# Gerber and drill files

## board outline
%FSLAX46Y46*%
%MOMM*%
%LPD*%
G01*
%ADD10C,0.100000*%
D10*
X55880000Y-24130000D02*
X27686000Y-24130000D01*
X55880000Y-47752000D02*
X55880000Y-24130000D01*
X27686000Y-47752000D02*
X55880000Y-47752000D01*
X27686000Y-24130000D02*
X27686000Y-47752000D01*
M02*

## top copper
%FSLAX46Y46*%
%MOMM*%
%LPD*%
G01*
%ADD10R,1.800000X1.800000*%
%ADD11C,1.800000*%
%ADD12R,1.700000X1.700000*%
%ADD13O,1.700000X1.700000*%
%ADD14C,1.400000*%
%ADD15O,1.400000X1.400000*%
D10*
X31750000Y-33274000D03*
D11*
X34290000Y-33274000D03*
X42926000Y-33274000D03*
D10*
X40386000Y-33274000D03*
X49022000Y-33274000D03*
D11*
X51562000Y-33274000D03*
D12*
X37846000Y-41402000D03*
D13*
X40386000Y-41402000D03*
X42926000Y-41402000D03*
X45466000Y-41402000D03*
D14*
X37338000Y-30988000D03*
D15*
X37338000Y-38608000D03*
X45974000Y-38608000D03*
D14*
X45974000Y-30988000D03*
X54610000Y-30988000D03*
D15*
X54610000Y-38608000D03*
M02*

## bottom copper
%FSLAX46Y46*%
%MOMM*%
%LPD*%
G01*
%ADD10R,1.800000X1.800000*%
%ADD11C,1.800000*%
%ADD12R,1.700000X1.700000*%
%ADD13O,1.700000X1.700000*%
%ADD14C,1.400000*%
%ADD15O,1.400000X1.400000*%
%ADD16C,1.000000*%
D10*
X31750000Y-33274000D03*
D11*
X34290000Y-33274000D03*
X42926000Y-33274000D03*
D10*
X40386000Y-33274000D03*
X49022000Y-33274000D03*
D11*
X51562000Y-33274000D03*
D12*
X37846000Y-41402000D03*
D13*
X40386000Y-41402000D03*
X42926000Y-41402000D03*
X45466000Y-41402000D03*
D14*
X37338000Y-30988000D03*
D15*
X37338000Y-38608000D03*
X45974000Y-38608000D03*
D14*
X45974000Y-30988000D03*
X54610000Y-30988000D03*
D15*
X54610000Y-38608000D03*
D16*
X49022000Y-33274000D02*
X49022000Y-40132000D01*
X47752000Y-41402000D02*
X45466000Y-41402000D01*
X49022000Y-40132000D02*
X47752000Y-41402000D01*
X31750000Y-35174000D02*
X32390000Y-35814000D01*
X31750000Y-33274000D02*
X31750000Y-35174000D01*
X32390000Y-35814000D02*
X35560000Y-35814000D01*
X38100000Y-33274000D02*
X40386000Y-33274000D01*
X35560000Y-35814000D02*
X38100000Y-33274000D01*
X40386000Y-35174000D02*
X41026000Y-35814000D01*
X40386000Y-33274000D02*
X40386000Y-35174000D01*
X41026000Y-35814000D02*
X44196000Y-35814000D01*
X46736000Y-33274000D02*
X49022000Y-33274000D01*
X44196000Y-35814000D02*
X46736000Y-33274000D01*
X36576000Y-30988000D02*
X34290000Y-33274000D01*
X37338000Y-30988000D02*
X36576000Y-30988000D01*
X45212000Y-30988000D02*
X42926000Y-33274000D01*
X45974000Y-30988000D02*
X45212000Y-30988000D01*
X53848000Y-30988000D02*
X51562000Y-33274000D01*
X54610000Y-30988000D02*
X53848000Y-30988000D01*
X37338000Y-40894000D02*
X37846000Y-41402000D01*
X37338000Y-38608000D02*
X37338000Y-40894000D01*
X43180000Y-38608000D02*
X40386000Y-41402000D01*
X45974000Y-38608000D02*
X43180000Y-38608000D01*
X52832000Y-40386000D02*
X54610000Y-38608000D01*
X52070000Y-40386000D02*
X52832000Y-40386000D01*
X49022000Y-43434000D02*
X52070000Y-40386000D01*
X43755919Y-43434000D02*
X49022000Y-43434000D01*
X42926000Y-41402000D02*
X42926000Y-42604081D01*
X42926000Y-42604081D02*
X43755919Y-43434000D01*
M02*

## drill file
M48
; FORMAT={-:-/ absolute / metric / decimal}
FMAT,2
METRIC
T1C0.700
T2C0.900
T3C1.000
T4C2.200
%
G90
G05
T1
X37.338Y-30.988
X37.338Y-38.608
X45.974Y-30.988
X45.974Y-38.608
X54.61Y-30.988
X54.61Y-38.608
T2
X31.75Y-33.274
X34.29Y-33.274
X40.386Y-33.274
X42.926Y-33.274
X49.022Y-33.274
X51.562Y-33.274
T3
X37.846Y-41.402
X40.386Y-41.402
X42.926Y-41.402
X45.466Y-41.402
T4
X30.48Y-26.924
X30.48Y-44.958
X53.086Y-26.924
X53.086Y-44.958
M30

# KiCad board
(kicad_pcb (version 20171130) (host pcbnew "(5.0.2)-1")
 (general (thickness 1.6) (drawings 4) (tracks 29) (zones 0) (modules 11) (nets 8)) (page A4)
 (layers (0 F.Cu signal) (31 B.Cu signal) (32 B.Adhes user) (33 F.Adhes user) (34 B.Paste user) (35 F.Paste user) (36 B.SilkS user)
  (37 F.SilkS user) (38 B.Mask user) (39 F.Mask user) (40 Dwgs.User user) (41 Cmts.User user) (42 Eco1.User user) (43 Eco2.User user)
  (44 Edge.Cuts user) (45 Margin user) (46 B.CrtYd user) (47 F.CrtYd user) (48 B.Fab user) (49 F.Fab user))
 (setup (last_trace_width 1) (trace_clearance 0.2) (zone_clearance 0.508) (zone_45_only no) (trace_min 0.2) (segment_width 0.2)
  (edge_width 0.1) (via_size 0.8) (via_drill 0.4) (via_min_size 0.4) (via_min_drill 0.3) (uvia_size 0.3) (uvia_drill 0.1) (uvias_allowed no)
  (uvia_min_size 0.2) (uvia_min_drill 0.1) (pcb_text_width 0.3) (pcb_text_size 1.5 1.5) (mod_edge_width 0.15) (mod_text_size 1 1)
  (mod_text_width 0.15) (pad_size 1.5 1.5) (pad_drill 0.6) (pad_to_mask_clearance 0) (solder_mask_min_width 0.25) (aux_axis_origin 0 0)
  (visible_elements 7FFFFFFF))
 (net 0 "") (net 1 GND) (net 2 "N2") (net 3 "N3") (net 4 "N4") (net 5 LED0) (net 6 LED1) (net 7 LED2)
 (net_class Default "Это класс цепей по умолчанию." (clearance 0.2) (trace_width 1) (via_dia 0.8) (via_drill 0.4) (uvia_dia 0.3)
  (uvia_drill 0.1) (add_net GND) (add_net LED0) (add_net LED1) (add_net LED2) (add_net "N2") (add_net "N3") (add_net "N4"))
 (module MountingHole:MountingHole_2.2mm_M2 (layer F.Cu) (at 53.086 26.924)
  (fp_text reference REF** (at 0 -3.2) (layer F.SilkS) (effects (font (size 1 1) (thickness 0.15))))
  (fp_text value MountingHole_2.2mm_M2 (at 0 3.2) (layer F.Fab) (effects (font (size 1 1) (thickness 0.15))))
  (pad 1 np_thru_hole circle (at 0 0) (size 2.2 2.2) (drill 2.2) (layers *.Cu *.Mask)))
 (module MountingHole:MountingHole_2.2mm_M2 (layer F.Cu) (at 30.48 26.924)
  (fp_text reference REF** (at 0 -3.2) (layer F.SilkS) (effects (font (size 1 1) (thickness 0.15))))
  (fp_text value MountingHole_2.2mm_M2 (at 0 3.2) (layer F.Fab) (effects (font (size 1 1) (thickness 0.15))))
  (pad 1 np_thru_hole circle (at 0 0) (size 2.2 2.2) (drill 2.2) (layers *.Cu *.Mask)))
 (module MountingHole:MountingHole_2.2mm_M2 (layer F.Cu) (at 53.086 44.958)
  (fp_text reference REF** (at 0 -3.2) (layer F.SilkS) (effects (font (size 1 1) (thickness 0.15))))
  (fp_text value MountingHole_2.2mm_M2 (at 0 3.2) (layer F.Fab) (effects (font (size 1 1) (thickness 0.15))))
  (pad 1 np_thru_hole circle (at 0 0) (size 2.2 2.2) (drill 2.2) (layers *.Cu *.Mask)))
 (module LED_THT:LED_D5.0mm (layer F.Cu) (at 31.75 33.274)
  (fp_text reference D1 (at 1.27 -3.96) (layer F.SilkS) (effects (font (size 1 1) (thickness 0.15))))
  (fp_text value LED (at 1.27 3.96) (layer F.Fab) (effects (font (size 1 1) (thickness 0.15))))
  (pad 1 thru_hole rect (at 0 0) (size 1.8 1.8) (drill 0.9) (layers *.Cu *.Mask) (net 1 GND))
  (pad 2 thru_hole circle (at 2.54 0) (size 1.8 1.8) (drill 0.9) (layers *.Cu *.Mask) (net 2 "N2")))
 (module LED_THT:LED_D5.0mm (layer F.Cu) (at 40.386 33.274)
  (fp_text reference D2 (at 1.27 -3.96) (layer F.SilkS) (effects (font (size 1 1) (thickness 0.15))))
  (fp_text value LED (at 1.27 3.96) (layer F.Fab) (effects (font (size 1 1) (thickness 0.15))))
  (pad 2 thru_hole circle (at 2.54 0) (size 1.8 1.8) (drill 0.9) (layers *.Cu *.Mask) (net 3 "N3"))
  (pad 1 thru_hole rect (at 0 0) (size 1.8 1.8) (drill 0.9) (layers *.Cu *.Mask) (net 1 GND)))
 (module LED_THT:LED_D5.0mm (layer F.Cu) (at 49.022 33.274)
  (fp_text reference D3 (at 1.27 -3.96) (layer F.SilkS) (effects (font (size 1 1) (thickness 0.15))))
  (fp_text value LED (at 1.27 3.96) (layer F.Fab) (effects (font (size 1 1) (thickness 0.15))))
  (pad 1 thru_hole rect (at 0 0) (size 1.8 1.8) (drill 0.9) (layers *.Cu *.Mask) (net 1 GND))
  (pad 2 thru_hole circle (at 2.54 0) (size 1.8 1.8) (drill 0.9) (layers *.Cu *.Mask) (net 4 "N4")))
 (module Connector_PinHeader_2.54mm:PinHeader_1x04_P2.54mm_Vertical (layer F.Cu) (at 37.846 41.402 90)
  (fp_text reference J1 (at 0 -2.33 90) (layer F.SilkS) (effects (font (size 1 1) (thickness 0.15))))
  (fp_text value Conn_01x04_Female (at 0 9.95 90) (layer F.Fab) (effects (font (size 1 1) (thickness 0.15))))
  (pad 1 thru_hole rect (at 0 0 90) (size 1.7 1.7) (drill 1) (layers *.Cu *.Mask) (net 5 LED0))
  (pad 2 thru_hole oval (at 0 2.54 90) (size 1.7 1.7) (drill 1) (layers *.Cu *.Mask) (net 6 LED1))
  (pad 3 thru_hole oval (at 0 5.08 90) (size 1.7 1.7) (drill 1) (layers *.Cu *.Mask) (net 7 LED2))
  (pad 4 thru_hole oval (at 0 7.62 90) (size 1.7 1.7) (drill 1) (layers *.Cu *.Mask) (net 1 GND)))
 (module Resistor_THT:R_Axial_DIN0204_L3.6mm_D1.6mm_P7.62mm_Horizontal (layer F.Cu) (at 37.338 30.988 270)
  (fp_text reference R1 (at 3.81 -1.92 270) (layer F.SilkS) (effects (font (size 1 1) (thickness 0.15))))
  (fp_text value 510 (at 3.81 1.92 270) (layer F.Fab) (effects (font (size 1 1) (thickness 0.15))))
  (pad 1 thru_hole circle (at 0 0 270) (size 1.4 1.4) (drill 0.7) (layers *.Cu *.Mask) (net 2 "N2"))
  (pad 2 thru_hole oval (at 7.62 0 270) (size 1.4 1.4) (drill 0.7) (layers *.Cu *.Mask) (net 5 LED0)))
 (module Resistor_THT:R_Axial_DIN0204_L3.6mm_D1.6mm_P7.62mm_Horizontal (layer F.Cu) (at 45.974 30.988 270)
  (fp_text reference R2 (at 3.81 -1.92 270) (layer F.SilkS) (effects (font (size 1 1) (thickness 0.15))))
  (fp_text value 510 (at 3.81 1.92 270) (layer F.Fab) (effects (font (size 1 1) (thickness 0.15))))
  (pad 2 thru_hole oval (at 7.62 0 270) (size 1.4 1.4) (drill 0.7) (layers *.Cu *.Mask) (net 6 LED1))
  (pad 1 thru_hole circle (at 0 0 270) (size 1.4 1.4) (drill 0.7) (layers *.Cu *.Mask) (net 3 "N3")))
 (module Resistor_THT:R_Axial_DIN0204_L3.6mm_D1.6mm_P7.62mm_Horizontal (layer F.Cu) (at 54.61 30.988 270)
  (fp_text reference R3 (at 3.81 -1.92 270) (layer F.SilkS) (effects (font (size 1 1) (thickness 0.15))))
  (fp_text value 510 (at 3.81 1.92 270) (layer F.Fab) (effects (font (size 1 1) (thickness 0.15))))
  (pad 1 thru_hole circle (at 0 0 270) (size 1.4 1.4) (drill 0.7) (layers *.Cu *.Mask) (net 4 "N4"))
  (pad 2 thru_hole oval (at 7.62 0 270) (size 1.4 1.4) (drill 0.7) (layers *.Cu *.Mask) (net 7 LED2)))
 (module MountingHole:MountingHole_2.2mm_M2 (layer F.Cu) (at 30.48 44.958)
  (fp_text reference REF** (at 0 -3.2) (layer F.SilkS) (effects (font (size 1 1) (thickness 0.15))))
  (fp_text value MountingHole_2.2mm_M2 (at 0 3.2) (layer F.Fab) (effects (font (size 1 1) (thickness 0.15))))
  (pad 1 np_thru_hole circle (at 0 0) (size 2.2 2.2) (drill 2.2) (layers *.Cu *.Mask)))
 (gr_line (start 55.88 24.13) (end 27.686 24.13) (layer Edge.Cuts) (width 0.1))
 (gr_line (start 55.88 47.752) (end 55.88 24.13) (layer Edge.Cuts) (width 0.1))
 (gr_line (start 27.686 47.752) (end 55.88 47.752) (layer Edge.Cuts) (width 0.1))
 (gr_line (start 27.686 24.13) (end 27.686 47.752) (layer Edge.Cuts) (width 0.1))
 (segment (start 49.022 33.274) (end 49.022 40.132) (width 1) (layer B.Cu) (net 1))
 (segment (start 47.752 41.402) (end 45.466 41.402) (width 1) (layer B.Cu) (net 1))
 (segment (start 49.022 40.132) (end 47.752 41.402) (width 1) (layer B.Cu) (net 1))
 (segment (start 31.75 35.174) (end 32.39 35.814) (width 1) (layer B.Cu) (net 1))
 (segment (start 31.75 33.274) (end 31.75 35.174) (width 1) (layer B.Cu) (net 1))
 (segment (start 32.39 35.814) (end 35.56 35.814) (width 1) (layer B.Cu) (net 1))
 (segment (start 38.1 33.274) (end 40.386 33.274) (width 1) (layer B.Cu) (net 1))
 (segment (start 35.56 35.814) (end 38.1 33.274) (width 1) (layer B.Cu) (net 1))
 (segment (start 40.386 35.174) (end 41.026 35.814) (width 1) (layer B.Cu) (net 1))
 (segment (start 40.386 33.274) (end 40.386 35.174) (width 1) (layer B.Cu) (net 1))
 (segment (start 41.026 35.814) (end 44.196 35.814) (width 1) (layer B.Cu) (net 1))
 (segment (start 46.736 33.274) (end 49.022 33.274) (width 1) (layer B.Cu) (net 1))
 (segment (start 44.196 35.814) (end 46.736 33.274) (width 1) (layer B.Cu) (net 1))
 (segment (start 36.576 30.988) (end 34.29 33.274) (width 1) (layer B.Cu) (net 2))
 (segment (start 37.338 30.988) (end 36.576 30.988) (width 1) (layer B.Cu) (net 2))
 (segment (start 45.212 30.988) (end 42.926 33.274) (width 1) (layer B.Cu) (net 3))
 (segment (start 45.974 30.988) (end 45.212 30.988) (width 1) (layer B.Cu) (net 3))
 (segment (start 53.848 30.988) (end 51.562 33.274) (width 1) (layer B.Cu) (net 4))
 (segment (start 54.61 30.988) (end 53.848 30.988) (width 1) (layer B.Cu) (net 4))
 (segment (start 37.338 40.894) (end 37.846 41.402) (width 1) (layer B.Cu) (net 5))
 (segment (start 37.338 38.608) (end 37.338 40.894) (width 1) (layer B.Cu) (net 5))
 (segment (start 43.18 38.608) (end 40.386 41.402) (width 1) (layer B.Cu) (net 6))
 (segment (start 45.974 38.608) (end 43.18 38.608) (width 1) (layer B.Cu) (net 6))
 (segment (start 52.832 40.386) (end 54.61 38.608) (width 1) (layer B.Cu) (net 7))
 (segment (start 52.07 40.386) (end 52.832 40.386) (width 1) (layer B.Cu) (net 7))
 (segment (start 49.022 43.434) (end 52.07 40.386) (width 1) (layer B.Cu) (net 7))
 (segment (start 43.755919 43.434) (end 49.022 43.434) (width 1) (layer B.Cu) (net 7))
 (segment (start 42.926 41.402) (end 42.926 42.604081) (width 1) (layer B.Cu) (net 7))
 (segment (start 42.926 42.604081) (end 43.755919 43.434) (width 1) (layer B.Cu) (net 7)))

